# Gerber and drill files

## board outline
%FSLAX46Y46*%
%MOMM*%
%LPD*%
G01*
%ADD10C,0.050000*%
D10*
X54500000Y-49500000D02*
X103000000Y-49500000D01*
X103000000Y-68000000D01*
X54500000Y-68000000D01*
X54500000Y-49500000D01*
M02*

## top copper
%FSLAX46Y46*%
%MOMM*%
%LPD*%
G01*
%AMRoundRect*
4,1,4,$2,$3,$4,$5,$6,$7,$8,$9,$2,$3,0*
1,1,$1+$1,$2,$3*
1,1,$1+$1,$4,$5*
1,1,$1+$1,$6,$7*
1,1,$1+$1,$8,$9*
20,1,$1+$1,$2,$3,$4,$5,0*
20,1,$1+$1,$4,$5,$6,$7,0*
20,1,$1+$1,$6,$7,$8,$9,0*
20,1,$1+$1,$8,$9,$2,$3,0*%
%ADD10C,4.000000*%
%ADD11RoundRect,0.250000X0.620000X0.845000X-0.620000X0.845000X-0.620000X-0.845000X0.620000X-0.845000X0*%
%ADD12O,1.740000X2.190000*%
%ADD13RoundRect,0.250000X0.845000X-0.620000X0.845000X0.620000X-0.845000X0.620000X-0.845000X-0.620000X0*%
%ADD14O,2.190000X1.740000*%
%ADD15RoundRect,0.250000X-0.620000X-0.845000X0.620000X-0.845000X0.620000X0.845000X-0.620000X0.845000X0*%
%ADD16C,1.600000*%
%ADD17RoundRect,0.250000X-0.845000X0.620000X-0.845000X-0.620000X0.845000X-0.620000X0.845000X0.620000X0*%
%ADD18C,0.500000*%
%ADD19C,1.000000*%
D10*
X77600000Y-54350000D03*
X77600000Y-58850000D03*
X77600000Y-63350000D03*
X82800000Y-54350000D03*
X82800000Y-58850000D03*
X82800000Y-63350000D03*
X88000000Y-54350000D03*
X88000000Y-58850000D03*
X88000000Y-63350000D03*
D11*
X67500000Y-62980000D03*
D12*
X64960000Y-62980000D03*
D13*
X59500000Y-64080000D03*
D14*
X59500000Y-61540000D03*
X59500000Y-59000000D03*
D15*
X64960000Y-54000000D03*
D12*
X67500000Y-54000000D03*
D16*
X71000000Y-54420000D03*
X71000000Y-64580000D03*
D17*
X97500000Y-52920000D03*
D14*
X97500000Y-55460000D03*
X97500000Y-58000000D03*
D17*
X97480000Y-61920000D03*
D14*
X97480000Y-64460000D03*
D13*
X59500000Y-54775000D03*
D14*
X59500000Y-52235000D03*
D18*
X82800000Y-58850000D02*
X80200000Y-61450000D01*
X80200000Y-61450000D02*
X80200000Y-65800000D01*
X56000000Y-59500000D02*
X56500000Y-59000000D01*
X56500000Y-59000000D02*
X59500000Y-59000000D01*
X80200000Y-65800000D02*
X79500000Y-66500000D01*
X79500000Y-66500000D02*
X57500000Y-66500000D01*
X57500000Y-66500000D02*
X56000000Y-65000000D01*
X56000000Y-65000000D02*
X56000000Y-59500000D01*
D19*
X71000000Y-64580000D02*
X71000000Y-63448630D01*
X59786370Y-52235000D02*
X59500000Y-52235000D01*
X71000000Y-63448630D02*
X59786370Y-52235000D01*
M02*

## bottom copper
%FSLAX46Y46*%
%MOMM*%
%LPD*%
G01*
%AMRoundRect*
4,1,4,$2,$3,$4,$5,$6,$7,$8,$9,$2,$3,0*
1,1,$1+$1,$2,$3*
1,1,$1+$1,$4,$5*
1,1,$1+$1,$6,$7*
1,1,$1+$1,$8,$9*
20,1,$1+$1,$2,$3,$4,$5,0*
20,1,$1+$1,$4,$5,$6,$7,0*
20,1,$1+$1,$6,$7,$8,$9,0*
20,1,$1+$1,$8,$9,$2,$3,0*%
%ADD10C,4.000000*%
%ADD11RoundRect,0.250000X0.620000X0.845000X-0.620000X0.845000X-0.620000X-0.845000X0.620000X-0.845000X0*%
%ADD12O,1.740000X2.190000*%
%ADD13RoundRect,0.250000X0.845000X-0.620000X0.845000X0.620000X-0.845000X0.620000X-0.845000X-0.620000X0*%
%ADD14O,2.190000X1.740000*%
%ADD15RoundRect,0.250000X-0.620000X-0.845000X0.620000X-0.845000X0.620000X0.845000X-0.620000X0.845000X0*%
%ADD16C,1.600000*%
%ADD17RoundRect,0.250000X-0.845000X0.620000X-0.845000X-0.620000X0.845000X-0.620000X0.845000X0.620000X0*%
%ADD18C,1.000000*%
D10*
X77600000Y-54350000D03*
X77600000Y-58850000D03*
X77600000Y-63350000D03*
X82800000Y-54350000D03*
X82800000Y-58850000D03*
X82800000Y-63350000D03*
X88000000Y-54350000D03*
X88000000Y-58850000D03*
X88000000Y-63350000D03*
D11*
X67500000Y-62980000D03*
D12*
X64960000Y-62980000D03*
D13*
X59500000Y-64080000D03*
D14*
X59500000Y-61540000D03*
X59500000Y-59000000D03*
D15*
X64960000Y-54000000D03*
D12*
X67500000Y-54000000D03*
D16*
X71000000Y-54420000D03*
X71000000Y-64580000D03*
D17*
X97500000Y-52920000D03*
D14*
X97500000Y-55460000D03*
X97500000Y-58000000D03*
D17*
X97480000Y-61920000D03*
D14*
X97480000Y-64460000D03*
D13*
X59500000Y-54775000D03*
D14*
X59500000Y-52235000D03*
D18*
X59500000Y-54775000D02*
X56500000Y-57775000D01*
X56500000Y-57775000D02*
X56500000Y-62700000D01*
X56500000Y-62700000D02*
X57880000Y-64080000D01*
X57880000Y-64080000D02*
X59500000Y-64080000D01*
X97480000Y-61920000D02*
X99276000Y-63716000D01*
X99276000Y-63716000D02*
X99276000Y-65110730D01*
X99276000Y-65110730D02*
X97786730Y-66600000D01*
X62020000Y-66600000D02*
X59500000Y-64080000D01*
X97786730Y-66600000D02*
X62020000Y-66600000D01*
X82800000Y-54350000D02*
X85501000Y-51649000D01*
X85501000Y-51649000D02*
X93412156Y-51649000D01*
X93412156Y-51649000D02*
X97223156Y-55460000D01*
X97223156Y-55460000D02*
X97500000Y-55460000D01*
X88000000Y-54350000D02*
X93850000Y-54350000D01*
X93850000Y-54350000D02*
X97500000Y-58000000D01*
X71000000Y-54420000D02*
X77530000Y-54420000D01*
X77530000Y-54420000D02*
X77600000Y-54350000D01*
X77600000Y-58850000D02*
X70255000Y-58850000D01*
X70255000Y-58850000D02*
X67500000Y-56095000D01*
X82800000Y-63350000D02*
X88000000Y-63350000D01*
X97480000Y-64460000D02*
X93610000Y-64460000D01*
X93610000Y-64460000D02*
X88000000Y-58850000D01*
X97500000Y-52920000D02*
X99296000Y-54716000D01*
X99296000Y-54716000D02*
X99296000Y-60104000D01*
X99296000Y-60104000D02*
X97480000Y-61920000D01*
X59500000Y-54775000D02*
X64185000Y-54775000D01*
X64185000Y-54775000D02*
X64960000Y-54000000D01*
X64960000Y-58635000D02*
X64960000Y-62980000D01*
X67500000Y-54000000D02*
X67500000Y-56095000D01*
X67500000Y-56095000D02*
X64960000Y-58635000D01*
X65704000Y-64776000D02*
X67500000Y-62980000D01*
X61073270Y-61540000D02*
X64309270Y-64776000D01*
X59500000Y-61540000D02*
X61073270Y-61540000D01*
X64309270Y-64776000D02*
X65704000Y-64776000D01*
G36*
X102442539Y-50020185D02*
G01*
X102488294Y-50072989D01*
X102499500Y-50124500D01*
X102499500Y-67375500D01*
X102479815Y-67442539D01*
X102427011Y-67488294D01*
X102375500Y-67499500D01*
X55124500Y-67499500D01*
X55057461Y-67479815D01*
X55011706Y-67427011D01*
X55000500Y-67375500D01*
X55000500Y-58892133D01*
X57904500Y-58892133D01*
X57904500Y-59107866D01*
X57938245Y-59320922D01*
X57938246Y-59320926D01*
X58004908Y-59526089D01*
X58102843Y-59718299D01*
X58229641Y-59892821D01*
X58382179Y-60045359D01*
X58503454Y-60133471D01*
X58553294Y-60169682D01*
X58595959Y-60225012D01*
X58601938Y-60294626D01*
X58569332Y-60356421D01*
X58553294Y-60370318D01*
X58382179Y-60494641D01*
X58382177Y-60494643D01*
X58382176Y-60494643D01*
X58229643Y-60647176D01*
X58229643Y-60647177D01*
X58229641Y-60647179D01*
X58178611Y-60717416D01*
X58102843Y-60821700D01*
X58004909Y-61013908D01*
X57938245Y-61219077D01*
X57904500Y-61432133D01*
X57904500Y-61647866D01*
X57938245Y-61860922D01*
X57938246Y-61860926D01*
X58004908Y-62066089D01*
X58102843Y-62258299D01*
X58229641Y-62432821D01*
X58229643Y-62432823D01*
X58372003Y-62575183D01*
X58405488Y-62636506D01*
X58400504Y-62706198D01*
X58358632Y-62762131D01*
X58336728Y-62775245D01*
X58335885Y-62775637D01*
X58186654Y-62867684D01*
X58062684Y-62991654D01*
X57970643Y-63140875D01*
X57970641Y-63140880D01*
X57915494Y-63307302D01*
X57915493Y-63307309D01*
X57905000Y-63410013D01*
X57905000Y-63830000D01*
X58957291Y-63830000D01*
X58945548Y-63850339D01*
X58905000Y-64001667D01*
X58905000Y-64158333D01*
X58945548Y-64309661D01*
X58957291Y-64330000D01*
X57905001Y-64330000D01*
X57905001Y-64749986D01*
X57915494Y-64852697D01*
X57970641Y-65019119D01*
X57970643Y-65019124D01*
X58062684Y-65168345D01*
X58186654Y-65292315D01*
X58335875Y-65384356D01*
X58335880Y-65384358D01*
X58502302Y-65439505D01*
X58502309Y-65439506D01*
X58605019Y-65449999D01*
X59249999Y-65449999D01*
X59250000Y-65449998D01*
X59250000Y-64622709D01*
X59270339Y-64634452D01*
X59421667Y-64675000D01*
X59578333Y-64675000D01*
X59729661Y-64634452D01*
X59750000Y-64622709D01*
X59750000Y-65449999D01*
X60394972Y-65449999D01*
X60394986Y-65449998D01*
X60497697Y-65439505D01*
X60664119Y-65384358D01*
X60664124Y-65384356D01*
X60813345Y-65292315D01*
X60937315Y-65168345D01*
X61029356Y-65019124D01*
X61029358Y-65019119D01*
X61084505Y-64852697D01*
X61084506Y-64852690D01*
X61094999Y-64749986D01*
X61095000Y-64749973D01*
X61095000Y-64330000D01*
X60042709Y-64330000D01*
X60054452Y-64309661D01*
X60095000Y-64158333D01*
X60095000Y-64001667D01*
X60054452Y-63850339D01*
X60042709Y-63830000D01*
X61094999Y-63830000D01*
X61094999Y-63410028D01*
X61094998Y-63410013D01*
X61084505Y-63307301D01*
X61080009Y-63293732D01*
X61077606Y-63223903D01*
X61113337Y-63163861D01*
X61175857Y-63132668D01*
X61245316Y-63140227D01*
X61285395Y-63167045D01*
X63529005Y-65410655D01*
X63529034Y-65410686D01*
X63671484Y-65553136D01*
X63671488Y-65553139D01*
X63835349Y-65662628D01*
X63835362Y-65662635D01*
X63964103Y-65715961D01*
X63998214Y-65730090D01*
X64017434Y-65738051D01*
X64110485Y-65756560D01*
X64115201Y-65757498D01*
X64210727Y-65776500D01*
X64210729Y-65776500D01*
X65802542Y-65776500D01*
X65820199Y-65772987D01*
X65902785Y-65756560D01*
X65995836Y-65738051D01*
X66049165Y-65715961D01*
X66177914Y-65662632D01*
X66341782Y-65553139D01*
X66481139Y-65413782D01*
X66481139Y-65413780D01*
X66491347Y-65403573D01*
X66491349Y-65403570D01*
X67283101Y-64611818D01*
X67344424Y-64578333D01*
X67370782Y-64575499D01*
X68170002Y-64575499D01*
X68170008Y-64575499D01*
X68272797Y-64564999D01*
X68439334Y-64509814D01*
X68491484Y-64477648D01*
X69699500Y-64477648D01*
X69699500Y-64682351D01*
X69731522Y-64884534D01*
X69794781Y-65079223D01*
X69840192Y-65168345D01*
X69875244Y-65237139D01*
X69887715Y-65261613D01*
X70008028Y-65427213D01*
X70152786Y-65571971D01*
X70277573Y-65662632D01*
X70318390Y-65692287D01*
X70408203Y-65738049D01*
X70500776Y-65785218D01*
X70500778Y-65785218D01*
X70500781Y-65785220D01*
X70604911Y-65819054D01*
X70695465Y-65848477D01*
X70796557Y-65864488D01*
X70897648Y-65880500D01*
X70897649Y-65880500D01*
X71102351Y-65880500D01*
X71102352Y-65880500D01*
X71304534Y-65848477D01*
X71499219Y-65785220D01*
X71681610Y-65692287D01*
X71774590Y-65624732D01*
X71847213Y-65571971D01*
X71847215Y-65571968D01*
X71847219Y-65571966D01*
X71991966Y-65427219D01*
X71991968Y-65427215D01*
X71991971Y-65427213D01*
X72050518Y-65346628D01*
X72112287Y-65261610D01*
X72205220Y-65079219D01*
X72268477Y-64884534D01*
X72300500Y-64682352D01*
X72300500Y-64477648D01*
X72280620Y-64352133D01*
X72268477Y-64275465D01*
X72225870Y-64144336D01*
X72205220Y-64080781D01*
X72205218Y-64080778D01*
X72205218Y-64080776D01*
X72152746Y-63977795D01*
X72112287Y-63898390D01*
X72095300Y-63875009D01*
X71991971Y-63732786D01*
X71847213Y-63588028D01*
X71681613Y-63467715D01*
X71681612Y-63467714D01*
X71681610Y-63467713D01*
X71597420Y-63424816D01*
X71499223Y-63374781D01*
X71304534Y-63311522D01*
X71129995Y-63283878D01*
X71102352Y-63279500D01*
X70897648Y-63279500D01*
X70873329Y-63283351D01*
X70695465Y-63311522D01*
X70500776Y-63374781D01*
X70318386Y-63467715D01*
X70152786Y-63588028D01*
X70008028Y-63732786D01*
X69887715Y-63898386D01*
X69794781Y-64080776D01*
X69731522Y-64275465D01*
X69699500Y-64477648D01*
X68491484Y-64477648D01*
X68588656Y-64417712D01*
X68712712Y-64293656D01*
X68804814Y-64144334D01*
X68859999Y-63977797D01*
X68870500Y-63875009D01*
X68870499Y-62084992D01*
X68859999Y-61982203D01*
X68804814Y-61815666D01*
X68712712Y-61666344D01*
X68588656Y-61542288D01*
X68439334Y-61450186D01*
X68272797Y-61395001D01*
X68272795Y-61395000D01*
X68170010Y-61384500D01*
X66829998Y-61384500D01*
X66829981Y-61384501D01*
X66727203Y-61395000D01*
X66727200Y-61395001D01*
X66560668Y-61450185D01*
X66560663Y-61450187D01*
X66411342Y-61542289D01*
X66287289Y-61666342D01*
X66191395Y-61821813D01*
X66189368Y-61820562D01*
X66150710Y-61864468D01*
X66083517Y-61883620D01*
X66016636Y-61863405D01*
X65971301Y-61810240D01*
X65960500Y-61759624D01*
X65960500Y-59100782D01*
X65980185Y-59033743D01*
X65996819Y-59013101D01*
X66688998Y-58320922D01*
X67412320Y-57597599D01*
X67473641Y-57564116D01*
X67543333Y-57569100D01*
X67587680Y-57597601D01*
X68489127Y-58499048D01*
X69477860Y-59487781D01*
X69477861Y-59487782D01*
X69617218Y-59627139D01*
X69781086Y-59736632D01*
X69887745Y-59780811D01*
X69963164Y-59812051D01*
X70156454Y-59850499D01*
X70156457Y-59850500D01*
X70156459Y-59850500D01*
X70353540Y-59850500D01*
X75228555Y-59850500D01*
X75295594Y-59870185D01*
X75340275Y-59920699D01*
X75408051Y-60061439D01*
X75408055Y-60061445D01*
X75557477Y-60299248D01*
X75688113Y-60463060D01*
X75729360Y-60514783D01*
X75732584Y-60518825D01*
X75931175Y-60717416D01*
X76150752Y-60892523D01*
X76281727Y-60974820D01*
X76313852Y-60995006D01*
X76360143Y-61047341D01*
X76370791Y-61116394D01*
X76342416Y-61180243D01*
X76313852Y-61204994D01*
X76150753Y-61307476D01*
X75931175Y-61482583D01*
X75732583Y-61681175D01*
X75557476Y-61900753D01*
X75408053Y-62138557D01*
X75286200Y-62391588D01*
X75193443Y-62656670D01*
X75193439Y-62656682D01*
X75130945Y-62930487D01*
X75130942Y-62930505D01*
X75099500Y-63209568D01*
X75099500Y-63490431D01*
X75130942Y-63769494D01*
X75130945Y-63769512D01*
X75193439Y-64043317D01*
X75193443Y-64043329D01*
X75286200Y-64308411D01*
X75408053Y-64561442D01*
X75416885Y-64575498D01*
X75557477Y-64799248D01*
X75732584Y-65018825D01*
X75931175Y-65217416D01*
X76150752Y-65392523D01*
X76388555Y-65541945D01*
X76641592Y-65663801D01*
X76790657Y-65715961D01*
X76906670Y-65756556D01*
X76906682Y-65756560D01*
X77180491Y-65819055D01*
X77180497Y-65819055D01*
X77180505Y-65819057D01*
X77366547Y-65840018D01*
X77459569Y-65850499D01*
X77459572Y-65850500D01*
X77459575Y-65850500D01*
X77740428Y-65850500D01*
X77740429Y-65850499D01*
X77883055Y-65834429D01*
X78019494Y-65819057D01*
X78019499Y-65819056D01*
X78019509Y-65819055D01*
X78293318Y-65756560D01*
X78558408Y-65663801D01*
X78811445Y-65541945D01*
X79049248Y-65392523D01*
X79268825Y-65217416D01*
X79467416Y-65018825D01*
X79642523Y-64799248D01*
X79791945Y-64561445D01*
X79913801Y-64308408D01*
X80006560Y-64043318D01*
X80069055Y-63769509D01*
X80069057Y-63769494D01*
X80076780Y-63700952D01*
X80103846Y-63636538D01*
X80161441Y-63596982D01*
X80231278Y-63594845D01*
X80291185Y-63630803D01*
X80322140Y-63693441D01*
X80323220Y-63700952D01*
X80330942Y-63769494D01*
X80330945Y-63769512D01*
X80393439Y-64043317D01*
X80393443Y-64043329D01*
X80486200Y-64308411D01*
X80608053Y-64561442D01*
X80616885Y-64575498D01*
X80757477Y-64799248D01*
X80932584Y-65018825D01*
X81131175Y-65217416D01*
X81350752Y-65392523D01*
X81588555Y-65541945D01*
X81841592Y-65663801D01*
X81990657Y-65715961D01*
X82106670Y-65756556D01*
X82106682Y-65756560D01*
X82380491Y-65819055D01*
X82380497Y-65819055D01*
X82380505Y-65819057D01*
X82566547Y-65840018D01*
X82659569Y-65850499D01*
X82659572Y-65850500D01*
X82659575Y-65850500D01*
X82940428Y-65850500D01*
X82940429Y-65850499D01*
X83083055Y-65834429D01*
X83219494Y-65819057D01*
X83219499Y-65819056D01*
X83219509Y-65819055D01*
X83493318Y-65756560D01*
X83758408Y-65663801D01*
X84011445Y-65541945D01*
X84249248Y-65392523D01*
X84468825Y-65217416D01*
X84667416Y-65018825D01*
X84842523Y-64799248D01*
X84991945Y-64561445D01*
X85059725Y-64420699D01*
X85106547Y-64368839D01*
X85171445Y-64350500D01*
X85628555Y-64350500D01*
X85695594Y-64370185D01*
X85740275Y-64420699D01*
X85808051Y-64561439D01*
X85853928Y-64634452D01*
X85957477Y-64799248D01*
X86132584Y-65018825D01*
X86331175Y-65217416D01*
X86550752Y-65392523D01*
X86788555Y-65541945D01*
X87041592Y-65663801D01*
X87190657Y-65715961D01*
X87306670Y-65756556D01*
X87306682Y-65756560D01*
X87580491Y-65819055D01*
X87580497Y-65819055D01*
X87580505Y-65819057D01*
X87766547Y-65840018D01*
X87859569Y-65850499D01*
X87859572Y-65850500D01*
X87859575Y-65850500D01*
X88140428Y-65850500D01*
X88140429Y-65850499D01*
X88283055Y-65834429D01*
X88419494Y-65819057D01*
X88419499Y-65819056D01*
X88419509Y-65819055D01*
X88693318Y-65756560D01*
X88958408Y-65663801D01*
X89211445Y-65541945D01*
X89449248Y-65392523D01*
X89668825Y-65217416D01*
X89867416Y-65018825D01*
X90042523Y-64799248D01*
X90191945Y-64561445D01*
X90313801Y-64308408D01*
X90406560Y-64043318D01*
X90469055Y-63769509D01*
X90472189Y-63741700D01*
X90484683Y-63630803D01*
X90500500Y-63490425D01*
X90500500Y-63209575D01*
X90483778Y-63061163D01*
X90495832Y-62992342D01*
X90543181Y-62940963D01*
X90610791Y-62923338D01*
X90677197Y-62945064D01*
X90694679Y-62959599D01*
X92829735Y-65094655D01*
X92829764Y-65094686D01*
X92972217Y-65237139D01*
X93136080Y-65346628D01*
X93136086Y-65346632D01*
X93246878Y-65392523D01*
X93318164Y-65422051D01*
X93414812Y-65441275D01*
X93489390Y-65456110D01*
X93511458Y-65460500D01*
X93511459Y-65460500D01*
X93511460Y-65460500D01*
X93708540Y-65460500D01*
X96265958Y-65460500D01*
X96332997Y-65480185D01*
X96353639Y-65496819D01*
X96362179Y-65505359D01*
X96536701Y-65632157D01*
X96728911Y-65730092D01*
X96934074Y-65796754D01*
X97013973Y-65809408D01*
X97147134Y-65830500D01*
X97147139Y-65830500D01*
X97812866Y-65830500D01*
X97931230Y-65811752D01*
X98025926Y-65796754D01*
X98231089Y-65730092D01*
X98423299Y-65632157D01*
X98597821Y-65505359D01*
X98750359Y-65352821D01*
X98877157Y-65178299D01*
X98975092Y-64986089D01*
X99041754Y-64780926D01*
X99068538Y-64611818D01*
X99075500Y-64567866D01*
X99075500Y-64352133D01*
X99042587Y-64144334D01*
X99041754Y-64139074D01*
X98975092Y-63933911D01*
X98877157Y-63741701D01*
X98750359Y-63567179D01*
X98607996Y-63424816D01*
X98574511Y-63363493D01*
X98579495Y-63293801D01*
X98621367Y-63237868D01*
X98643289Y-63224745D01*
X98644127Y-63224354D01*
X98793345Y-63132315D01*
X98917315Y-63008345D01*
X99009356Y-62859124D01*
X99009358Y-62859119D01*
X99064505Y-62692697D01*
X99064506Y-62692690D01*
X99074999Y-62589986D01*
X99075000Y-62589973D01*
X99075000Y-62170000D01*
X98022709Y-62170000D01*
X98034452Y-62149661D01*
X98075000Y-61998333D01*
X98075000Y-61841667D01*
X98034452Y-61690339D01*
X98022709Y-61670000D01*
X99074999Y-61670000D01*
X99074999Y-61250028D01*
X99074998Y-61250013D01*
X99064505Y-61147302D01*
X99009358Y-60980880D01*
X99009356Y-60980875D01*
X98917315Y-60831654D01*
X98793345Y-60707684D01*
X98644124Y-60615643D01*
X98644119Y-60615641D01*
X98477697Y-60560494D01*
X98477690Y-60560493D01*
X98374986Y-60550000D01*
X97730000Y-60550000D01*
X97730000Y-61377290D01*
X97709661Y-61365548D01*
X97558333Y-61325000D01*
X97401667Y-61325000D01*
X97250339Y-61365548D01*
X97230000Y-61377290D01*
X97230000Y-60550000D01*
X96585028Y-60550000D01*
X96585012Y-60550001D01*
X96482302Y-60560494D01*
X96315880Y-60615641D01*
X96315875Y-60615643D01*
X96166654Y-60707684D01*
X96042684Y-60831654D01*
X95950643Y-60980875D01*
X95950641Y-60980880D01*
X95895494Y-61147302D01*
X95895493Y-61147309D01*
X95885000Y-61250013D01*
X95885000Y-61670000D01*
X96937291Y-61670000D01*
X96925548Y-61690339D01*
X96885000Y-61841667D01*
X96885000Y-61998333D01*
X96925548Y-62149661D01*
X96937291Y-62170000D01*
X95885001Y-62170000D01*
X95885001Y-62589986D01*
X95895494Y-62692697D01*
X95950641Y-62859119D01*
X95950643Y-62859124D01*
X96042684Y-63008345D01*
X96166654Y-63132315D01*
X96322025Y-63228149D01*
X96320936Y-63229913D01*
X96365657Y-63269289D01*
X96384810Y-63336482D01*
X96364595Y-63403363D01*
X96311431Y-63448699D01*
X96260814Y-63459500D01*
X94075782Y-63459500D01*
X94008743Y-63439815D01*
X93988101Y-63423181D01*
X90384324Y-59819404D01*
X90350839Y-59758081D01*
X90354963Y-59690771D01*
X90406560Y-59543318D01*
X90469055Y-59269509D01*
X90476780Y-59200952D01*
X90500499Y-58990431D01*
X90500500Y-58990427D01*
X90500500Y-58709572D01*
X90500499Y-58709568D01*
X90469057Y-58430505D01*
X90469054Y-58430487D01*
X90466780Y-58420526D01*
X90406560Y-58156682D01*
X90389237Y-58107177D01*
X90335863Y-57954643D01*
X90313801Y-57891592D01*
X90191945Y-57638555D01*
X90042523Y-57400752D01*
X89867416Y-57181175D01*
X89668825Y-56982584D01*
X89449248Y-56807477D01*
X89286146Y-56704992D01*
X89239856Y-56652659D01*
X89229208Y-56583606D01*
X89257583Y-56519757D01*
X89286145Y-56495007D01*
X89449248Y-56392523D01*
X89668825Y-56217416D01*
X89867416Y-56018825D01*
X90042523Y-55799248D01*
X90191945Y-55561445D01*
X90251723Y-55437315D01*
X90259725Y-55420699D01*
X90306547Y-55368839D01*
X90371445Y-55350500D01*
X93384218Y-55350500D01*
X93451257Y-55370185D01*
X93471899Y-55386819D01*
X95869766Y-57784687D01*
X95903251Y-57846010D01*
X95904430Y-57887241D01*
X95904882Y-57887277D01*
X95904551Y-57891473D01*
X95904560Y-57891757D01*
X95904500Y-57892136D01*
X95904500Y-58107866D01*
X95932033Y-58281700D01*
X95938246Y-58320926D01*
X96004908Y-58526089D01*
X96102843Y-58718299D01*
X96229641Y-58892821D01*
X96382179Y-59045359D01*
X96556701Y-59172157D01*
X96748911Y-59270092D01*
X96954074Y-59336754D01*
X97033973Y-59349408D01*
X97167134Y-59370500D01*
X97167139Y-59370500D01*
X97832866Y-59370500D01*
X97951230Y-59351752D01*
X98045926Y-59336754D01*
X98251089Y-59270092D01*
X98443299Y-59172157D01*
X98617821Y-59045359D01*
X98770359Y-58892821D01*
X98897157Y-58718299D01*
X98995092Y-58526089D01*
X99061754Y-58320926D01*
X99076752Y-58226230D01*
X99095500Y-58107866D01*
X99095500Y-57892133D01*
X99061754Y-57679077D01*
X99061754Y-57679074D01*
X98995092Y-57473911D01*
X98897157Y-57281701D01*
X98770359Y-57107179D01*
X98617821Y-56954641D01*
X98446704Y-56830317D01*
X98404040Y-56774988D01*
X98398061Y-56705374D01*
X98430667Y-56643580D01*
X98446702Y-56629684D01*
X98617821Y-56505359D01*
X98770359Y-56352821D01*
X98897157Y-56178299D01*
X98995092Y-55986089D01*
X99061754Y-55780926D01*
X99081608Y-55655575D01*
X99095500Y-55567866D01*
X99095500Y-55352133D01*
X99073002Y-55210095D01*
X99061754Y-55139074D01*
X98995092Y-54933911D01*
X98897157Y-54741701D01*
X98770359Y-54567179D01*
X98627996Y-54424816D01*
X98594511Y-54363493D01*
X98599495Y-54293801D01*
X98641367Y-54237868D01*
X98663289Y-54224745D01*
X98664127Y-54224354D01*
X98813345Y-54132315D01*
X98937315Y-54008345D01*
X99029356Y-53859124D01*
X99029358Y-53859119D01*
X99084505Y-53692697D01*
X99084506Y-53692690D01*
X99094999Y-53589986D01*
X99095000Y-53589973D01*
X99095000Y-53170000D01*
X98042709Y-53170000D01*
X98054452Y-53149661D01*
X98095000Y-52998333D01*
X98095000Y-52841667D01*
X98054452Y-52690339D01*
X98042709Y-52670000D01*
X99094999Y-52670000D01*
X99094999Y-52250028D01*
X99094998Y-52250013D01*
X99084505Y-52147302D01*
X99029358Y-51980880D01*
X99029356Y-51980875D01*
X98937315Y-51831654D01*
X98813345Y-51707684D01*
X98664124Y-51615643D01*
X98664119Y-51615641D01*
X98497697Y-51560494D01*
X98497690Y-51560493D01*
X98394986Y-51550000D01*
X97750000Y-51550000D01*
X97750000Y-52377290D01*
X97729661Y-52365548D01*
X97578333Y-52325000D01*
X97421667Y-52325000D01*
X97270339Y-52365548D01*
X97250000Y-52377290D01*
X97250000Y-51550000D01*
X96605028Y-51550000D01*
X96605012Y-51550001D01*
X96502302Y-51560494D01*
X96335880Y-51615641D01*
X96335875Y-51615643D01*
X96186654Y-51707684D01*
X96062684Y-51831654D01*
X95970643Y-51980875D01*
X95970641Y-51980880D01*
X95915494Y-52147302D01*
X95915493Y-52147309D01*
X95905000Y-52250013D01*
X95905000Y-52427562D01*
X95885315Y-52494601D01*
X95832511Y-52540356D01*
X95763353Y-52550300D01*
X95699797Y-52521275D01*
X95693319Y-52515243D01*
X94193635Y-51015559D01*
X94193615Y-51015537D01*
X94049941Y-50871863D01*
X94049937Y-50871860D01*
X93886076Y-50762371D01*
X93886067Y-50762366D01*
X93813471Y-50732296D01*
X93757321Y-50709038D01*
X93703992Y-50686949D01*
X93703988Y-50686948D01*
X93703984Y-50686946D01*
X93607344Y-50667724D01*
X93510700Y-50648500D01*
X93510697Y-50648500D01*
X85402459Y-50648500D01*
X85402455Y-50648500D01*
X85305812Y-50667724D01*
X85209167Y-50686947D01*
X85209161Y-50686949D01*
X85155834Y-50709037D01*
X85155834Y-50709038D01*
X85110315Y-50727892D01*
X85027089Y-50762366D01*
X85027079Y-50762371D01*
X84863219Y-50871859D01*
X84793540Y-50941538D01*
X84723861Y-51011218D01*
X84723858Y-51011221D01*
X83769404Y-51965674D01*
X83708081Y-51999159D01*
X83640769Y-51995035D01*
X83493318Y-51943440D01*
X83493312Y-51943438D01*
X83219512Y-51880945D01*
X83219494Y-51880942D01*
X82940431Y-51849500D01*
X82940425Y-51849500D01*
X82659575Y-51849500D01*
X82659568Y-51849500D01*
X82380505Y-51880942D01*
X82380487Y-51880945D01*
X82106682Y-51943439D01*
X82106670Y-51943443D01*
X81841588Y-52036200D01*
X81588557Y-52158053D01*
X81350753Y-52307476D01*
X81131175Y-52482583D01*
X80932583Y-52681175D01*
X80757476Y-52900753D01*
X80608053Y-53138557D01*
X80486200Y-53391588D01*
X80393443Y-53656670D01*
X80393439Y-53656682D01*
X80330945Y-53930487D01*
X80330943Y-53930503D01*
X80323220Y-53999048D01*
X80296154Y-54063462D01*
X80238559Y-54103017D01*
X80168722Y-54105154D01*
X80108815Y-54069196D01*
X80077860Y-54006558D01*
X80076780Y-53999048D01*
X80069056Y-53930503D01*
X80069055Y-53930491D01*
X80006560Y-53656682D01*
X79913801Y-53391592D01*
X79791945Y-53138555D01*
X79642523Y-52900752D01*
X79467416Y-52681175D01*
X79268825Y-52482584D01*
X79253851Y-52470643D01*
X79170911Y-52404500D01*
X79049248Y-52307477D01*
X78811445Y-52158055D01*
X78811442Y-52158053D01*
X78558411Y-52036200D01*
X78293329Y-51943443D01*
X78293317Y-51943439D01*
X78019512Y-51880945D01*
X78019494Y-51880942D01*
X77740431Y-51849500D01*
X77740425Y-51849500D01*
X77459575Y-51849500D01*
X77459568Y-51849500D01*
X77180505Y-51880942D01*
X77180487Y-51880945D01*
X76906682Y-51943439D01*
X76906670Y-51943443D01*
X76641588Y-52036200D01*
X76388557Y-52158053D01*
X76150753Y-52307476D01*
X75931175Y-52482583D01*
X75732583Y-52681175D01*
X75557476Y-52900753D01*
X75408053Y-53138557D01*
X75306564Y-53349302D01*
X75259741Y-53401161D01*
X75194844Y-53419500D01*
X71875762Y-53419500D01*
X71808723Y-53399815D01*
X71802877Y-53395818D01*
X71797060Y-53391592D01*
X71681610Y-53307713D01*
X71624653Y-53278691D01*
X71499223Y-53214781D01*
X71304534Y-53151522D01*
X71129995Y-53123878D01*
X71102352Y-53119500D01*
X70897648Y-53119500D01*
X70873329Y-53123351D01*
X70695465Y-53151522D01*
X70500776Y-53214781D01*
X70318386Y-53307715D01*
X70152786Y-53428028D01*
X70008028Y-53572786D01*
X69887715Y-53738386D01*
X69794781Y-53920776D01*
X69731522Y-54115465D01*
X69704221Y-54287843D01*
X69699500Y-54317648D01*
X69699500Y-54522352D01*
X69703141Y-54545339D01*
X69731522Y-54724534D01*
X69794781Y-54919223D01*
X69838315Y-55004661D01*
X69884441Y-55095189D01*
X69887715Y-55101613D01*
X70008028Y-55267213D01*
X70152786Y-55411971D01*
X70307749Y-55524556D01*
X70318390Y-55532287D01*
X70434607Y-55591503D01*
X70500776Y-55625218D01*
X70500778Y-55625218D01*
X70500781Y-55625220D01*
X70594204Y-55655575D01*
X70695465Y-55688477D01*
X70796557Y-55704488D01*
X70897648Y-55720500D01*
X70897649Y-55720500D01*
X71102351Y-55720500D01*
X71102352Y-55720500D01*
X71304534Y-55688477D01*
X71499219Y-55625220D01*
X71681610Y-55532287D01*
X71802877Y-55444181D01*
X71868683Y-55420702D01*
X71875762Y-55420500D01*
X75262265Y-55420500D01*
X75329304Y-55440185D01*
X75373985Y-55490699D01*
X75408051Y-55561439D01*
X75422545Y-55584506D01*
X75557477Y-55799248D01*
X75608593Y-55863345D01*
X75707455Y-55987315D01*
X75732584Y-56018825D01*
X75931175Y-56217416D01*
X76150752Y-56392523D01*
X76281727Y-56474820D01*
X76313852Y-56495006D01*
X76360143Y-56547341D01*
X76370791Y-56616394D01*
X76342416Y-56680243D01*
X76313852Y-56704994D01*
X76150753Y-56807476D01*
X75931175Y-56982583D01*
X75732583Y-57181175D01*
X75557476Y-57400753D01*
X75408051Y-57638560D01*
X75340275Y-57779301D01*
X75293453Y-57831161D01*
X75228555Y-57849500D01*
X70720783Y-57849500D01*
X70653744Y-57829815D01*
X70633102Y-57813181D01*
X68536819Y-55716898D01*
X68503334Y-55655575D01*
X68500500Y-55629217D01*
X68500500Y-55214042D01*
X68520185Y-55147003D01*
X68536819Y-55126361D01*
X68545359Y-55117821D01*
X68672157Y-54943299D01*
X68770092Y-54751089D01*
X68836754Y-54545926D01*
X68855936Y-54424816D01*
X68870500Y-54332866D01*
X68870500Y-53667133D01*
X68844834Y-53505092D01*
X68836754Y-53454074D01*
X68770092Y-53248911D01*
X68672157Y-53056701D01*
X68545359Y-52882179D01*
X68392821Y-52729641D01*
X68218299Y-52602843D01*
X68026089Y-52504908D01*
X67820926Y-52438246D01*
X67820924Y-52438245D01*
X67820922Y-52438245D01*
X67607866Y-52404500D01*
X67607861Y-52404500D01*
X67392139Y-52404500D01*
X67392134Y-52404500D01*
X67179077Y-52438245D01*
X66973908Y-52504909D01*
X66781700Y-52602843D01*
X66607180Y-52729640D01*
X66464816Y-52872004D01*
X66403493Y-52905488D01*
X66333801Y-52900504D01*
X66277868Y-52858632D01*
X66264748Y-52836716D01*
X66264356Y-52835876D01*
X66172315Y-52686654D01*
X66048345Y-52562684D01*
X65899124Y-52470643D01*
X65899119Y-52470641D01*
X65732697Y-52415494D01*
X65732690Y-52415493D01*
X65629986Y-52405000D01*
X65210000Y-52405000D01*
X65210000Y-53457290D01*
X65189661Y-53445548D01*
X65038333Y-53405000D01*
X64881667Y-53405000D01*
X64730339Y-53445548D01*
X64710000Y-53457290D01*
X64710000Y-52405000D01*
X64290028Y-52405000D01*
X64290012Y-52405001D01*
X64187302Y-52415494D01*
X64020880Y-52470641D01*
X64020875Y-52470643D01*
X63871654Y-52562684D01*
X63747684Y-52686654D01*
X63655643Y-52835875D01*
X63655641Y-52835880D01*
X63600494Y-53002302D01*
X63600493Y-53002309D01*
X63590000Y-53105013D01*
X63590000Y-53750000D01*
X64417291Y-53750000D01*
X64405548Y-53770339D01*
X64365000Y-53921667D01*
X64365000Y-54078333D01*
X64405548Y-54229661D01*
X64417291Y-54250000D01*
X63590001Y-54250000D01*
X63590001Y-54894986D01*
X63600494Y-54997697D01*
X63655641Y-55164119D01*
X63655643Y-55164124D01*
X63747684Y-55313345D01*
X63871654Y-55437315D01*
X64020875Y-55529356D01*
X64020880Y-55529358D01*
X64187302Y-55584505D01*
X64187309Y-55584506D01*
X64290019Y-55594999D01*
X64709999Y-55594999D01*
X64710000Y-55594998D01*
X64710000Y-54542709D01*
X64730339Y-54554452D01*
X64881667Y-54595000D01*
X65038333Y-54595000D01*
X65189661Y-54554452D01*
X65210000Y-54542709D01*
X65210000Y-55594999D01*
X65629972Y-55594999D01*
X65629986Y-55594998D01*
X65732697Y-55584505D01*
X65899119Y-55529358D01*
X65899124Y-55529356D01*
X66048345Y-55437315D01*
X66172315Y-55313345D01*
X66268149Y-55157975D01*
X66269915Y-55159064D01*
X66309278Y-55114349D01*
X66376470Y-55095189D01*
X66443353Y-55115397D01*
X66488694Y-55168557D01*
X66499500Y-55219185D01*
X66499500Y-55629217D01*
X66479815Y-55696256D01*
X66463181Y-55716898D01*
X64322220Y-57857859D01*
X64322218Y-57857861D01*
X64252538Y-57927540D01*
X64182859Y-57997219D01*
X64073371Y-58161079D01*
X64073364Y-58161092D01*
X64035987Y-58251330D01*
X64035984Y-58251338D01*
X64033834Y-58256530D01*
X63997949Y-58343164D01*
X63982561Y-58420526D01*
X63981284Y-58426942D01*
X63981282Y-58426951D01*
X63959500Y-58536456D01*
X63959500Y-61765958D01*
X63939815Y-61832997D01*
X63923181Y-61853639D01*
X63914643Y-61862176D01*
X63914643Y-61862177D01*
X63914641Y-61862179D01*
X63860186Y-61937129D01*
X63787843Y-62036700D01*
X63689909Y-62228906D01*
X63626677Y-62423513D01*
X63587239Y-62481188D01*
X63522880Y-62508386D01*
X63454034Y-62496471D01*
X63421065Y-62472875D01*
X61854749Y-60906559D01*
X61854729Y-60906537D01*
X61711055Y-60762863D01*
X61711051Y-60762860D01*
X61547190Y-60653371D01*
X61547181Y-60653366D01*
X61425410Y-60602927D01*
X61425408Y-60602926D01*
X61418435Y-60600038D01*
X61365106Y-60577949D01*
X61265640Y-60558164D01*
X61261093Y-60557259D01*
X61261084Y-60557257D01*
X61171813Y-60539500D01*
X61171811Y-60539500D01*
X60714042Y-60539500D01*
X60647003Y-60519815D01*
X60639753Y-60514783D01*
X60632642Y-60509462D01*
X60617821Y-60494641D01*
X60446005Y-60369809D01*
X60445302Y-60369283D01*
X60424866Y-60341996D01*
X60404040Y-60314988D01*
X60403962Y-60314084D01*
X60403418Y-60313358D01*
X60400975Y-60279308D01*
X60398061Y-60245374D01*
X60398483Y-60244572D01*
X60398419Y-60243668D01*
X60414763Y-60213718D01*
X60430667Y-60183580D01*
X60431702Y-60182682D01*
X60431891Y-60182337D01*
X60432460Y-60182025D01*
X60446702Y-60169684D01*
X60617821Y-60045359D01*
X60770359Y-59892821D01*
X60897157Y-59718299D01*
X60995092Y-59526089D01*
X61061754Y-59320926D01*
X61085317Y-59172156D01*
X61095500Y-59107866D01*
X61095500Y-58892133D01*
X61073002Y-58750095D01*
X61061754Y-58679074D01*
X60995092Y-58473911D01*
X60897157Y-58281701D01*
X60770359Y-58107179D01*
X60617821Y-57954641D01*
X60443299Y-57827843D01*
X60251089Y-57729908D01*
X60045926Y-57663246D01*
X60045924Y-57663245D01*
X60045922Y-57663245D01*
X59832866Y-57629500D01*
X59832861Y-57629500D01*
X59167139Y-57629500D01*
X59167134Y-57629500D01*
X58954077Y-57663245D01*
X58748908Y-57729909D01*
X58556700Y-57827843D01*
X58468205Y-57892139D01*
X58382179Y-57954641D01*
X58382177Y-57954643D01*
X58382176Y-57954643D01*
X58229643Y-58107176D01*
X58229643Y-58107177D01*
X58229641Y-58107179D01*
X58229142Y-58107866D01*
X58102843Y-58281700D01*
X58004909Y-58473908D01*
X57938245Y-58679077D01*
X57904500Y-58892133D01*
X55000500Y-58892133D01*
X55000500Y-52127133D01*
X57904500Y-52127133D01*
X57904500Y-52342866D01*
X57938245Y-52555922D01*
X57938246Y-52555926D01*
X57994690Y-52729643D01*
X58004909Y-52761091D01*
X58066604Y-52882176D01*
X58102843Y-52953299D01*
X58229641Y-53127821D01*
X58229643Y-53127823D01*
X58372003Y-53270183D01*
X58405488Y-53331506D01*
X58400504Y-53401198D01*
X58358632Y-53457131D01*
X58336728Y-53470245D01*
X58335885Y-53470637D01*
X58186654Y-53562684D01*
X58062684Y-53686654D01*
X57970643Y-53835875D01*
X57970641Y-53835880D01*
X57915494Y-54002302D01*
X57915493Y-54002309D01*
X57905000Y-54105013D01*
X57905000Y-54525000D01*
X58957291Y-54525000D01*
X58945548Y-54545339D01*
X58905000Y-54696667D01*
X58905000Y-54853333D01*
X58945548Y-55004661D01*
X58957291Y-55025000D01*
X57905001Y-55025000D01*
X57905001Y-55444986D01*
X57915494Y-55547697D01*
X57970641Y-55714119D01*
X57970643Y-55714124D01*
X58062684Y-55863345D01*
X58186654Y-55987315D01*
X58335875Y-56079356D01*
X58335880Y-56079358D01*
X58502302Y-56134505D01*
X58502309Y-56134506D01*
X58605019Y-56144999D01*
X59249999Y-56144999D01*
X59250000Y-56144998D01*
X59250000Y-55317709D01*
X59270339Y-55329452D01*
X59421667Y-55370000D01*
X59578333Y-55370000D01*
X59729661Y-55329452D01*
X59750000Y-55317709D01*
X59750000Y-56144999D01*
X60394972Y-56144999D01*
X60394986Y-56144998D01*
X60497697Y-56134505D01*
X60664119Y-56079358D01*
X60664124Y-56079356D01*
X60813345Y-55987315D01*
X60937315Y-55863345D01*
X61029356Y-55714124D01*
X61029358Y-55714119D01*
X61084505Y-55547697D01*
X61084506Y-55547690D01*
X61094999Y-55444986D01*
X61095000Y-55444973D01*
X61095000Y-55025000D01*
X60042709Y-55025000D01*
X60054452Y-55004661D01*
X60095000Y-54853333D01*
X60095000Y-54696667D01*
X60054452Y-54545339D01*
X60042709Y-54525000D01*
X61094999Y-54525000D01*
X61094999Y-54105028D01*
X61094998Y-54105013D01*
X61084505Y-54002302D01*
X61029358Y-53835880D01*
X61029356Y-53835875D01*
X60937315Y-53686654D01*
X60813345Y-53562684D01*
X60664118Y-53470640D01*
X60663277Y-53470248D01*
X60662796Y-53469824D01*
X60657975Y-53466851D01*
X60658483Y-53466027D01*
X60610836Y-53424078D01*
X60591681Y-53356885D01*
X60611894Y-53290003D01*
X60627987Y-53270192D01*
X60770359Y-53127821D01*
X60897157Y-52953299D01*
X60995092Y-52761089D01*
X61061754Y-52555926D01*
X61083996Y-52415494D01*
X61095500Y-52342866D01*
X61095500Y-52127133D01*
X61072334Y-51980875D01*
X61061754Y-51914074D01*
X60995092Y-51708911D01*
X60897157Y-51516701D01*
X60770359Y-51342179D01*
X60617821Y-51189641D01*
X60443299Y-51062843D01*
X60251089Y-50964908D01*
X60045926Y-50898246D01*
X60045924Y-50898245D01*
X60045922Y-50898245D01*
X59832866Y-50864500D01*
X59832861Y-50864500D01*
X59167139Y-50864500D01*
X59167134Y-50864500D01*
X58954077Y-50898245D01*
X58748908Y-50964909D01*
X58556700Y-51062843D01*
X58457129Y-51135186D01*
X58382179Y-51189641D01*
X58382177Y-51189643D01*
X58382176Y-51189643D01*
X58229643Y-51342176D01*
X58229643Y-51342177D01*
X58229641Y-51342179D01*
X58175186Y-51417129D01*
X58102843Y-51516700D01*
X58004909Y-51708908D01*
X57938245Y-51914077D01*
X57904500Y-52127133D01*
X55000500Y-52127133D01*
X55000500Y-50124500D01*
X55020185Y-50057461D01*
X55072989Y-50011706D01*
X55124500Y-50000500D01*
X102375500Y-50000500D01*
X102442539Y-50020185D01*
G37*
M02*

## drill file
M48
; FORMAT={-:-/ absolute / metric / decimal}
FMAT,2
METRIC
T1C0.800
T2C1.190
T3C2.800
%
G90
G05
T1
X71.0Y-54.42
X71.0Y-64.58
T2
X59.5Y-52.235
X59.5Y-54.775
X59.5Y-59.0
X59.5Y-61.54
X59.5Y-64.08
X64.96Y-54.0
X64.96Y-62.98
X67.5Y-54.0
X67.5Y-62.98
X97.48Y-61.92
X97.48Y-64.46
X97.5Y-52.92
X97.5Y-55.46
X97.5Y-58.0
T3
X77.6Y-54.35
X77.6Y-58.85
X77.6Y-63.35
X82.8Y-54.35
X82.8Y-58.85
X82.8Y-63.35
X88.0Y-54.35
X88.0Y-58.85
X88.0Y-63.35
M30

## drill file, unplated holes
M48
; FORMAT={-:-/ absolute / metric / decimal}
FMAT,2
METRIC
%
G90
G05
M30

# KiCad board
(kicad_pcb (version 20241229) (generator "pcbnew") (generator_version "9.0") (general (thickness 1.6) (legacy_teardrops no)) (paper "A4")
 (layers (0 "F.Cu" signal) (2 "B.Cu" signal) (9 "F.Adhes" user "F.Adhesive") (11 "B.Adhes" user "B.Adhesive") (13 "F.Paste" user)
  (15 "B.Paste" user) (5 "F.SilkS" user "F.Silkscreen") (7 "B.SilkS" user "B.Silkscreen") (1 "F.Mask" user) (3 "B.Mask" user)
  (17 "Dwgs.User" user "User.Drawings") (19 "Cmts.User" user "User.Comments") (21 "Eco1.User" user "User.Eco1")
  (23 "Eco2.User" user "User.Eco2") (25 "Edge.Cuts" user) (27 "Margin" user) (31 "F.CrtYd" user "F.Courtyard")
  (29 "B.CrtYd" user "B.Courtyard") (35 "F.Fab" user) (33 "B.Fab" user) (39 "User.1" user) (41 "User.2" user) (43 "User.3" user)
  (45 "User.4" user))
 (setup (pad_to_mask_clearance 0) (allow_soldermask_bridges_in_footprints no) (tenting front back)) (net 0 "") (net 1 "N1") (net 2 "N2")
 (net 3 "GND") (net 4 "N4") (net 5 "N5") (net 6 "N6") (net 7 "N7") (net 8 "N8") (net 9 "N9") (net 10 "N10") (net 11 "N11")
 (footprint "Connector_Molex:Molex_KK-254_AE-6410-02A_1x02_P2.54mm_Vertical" (layer "F.Cu") (at 67.5 62.98 180)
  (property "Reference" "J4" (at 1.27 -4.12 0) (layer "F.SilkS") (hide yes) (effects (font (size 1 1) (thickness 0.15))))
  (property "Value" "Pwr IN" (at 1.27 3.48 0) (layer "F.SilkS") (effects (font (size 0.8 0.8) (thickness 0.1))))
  (pad "1" thru_hole roundrect (at 0 0 180) (size 1.74 2.19) (drill 1.19) (layers "*.Cu" "*.Mask") (remove_unused_layers no)
   (roundrect_rratio 0.143678) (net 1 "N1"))
  (pad "2" thru_hole oval (at 2.54 0 180) (size 1.74 2.19) (drill 1.19) (layers "*.Cu" "*.Mask") (remove_unused_layers no) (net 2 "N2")))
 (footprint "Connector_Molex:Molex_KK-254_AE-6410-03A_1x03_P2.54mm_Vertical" (layer "F.Cu") (at 59.5 64.08 90)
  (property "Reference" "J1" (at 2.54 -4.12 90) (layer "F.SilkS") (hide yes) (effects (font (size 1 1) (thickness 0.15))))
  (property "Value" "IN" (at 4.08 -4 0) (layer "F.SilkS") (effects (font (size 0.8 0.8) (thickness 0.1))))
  (pad "1" thru_hole roundrect (at 0 0 90) (size 1.74 2.19) (drill 1.19) (layers "*.Cu" "*.Mask") (remove_unused_layers no)
   (roundrect_rratio 0.143678) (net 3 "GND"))
  (pad "2" thru_hole oval (at 2.54 0 90) (size 1.74 2.19) (drill 1.19) (layers "*.Cu" "*.Mask") (remove_unused_layers no) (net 1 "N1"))
  (pad "3" thru_hole oval (at 5.08 0 90) (size 1.74 2.19) (drill 1.19) (layers "*.Cu" "*.Mask") (remove_unused_layers no) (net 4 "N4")))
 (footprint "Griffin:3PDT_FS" (layer "F.Cu") (at 80.6 57.85)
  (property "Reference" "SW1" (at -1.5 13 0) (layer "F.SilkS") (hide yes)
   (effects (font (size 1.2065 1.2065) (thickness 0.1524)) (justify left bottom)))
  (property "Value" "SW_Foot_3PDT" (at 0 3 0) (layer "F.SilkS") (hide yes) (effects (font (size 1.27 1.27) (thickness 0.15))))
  (pad "A1" thru_hole circle (at -3 -3.5 180) (size 4 4) (drill 2.8) (layers "*.Cu" "*.Mask") (remove_unused_layers no) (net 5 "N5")
   (solder_mask_margin 0.1016))
  (pad "A2" thru_hole circle (at -3 1 180) (size 4 4) (drill 2.8) (layers "*.Cu" "*.Mask") (remove_unused_layers no) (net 2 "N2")
   (solder_mask_margin 0.1016))
  (pad "A3" thru_hole circle (at -3 5.5 180) (size 4 4) (drill 2.8) (layers "*.Cu" "*.Mask") (remove_unused_layers no) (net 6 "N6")
   (solder_mask_margin 0.1016))
  (pad "B1" thru_hole circle (at 2.2 -3.5 180) (size 4 4) (drill 2.8) (layers "*.Cu" "*.Mask") (remove_unused_layers no) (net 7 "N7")
   (solder_mask_margin 0.1016))
  (pad "B2" thru_hole circle (at 2.2 1 180) (size 4 4) (drill 2.8) (layers "*.Cu" "*.Mask") (remove_unused_layers no) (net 4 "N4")
   (solder_mask_margin 0.1016))
  (pad "B3" thru_hole circle (at 2.2 5.5 180) (size 4 4) (drill 2.8) (layers "*.Cu" "*.Mask") (remove_unused_layers no) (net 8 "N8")
   (solder_mask_margin 0.1016))
  (pad "C1" thru_hole circle (at 7.4 -3.5 180) (size 4 4) (drill 2.8) (layers "*.Cu" "*.Mask") (remove_unused_layers no) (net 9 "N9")
   (solder_mask_margin 0.1016))
  (pad "C2" thru_hole circle (at 7.4 1 180) (size 4 4) (drill 2.8) (layers "*.Cu" "*.Mask") (remove_unused_layers no) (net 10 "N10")
   (solder_mask_margin 0.1016))
  (pad "C3" thru_hole circle (at 7.4 5.5 180) (size 4 4) (drill 2.8) (layers "*.Cu" "*.Mask") (remove_unused_layers no) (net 8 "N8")
   (solder_mask_margin 0.1016)))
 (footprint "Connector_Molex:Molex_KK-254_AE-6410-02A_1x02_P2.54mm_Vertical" (layer "F.Cu") (at 64.96 54)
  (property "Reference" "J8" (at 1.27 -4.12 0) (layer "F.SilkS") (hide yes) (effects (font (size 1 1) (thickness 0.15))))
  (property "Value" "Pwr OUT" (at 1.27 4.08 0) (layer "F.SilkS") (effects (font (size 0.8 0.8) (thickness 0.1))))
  (pad "1" thru_hole roundrect (at 0 0) (size 1.74 2.19) (drill 1.19) (layers "*.Cu" "*.Mask") (remove_unused_layers no)
   (roundrect_rratio 0.143678) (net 3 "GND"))
  (pad "2" thru_hole oval (at 2.54 0) (size 1.74 2.19) (drill 1.19) (layers "*.Cu" "*.Mask") (remove_unused_layers no) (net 2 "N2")))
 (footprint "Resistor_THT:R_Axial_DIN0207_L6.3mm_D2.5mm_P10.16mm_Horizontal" (layer "F.Cu") (at 71 54.42 -90)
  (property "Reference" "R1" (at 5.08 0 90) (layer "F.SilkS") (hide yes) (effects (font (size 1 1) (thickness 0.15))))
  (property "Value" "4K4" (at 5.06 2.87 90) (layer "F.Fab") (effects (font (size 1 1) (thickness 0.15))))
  (pad "1" thru_hole circle (at 0 0 270) (size 1.6 1.6) (drill 0.8) (layers "*.Cu" "*.Mask") (remove_unused_layers no) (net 5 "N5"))
  (pad "2" thru_hole circle (at 10.16 0 270) (size 1.6 1.6) (drill 0.8) (layers "*.Cu" "*.Mask") (remove_unused_layers no) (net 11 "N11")))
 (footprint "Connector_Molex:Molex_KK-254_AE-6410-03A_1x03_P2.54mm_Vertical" (layer "F.Cu") (at 97.5 52.92 -90)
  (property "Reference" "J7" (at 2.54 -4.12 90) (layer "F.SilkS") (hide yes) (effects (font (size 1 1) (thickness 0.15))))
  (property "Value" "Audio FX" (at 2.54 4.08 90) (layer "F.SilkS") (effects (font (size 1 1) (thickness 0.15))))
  (pad "1" thru_hole roundrect (at 0 0 270) (size 1.74 2.19) (drill 1.19) (layers "*.Cu" "*.Mask") (remove_unused_layers no)
   (roundrect_rratio 0.143678) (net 3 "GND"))
  (pad "2" thru_hole oval (at 2.54 0 270) (size 1.74 2.19) (drill 1.19) (layers "*.Cu" "*.Mask") (remove_unused_layers no) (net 7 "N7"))
  (pad "3" thru_hole oval (at 5.08 0 270) (size 1.74 2.19) (drill 1.19) (layers "*.Cu" "*.Mask") (remove_unused_layers no) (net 9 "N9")))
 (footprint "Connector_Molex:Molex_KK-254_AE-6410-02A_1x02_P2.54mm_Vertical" (layer "F.Cu") (at 97.48 61.92 -90)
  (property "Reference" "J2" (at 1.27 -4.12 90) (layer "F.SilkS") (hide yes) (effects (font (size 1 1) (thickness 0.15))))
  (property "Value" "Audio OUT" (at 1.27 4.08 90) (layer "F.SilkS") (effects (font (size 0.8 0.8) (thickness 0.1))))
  (pad "1" thru_hole roundrect (at 0 0 270) (size 1.74 2.19) (drill 1.19) (layers "*.Cu" "*.Mask") (remove_unused_layers no)
   (roundrect_rratio 0.143678) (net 3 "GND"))
  (pad "2" thru_hole oval (at 2.54 0 270) (size 1.74 2.19) (drill 1.19) (layers "*.Cu" "*.Mask") (remove_unused_layers no) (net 10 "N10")))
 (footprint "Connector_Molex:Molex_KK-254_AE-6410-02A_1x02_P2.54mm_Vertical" (layer "F.Cu") (at 59.5 54.775 90)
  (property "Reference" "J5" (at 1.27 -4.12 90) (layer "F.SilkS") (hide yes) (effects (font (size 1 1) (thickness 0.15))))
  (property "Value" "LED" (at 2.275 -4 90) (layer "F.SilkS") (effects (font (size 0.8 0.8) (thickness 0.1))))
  (pad "1" thru_hole roundrect (at 0 0 90) (size 1.74 2.19) (drill 1.19) (layers "*.Cu" "*.Mask") (remove_unused_layers no)
   (roundrect_rratio 0.143678) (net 3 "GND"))
  (pad "2" thru_hole oval (at 2.54 0 90) (size 1.74 2.19) (drill 1.19) (layers "*.Cu" "*.Mask") (remove_unused_layers no) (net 11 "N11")))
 (gr_rect (start 54.5 49.5) (end 103 68) (stroke (width 0.05) (type default)) (fill no) (layer "Edge.Cuts"))
 (segment (start 97.5 52.92) (end 99.296 54.716) (width 1) (layer "B.Cu") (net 3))
 (segment (start 59.5 54.775) (end 56.5 57.775) (width 1) (layer "B.Cu") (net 3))
 (segment (start 59.5 54.775) (end 64.185 54.775) (width 1) (layer "B.Cu") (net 3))
 (segment (start 97.78673 66.6) (end 62.02 66.6) (width 1) (layer "B.Cu") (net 3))
 (segment (start 57.88 64.08) (end 59.5 64.08) (width 1) (layer "B.Cu") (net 3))
 (segment (start 99.296 60.104) (end 97.48 61.92) (width 1) (layer "B.Cu") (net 3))
 (segment (start 56.5 62.7) (end 57.88 64.08) (width 1) (layer "B.Cu") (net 3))
 (segment (start 99.296 54.716) (end 99.296 60.104) (width 1) (layer "B.Cu") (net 3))
 (segment (start 62.02 66.6) (end 59.5 64.08) (width 1) (layer "B.Cu") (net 3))
 (segment (start 97.48 61.92) (end 99.276 63.716) (width 1) (layer "B.Cu") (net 3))
 (segment (start 99.276 65.11073) (end 97.78673 66.6) (width 1) (layer "B.Cu") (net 3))
 (segment (start 56.5 57.775) (end 56.5 62.7) (width 1) (layer "B.Cu") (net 3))
 (segment (start 64.185 54.775) (end 64.96 54) (width 1) (layer "B.Cu") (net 3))
 (segment (start 99.276 63.716) (end 99.276 65.11073) (width 1) (layer "B.Cu") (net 3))
 (segment (start 64.96 58.635) (end 64.96 62.98) (width 1) (layer "B.Cu") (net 2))
 (segment (start 67.5 54) (end 67.5 56.095) (width 1) (layer "B.Cu") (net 2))
 (segment (start 70.255 58.85) (end 67.5 56.095) (width 1) (layer "B.Cu") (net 2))
 (segment (start 67.5 56.095) (end 64.96 58.635) (width 1) (layer "B.Cu") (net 2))
 (segment (start 77.6 58.85) (end 70.255 58.85) (width 1) (layer "B.Cu") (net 2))
 (segment (start 71 64.58) (end 71 63.44863) (width 1) (layer "F.Cu") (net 11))
 (segment (start 59.78637 52.235) (end 59.5 52.235) (width 1) (layer "F.Cu") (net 11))
 (segment (start 71 63.44863) (end 59.78637 52.235) (width 1) (layer "F.Cu") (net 11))
 (segment (start 97.223156 55.46) (end 97.5 55.46) (width 1) (layer "B.Cu") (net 7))
 (segment (start 85.501 51.649) (end 93.412156 51.649) (width 1) (layer "B.Cu") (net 7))
 (segment (start 93.412156 51.649) (end 97.223156 55.46) (width 1) (layer "B.Cu") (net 7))
 (segment (start 82.8 54.35) (end 85.501 51.649) (width 1) (layer "B.Cu") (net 7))
 (segment (start 77.53 54.42) (end 77.6 54.35) (width 1) (layer "B.Cu") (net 5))
 (segment (start 71 54.42) (end 77.53 54.42) (width 1) (layer "B.Cu") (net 5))
 (segment (start 82.8 58.85) (end 80.2 61.45) (width 0.5) (layer "F.Cu") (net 4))
 (segment (start 56 59.5) (end 56.5 59) (width 0.5) (layer "F.Cu") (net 4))
 (segment (start 56.5 59) (end 59.5 59) (width 0.5) (layer "F.Cu") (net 4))
 (segment (start 57.5 66.5) (end 56 65) (width 0.5) (layer "F.Cu") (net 4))
 (segment (start 79.5 66.5) (end 57.5 66.5) (width 0.5) (layer "F.Cu") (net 4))
 (segment (start 80.2 65.8) (end 79.5 66.5) (width 0.5) (layer "F.Cu") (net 4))
 (segment (start 80.2 61.45) (end 80.2 65.8) (width 0.5) (layer "F.Cu") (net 4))
 (segment (start 56 65) (end 56 59.5) (width 0.5) (layer "F.Cu") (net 4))
 (segment (start 65.704 64.776) (end 67.5 62.98) (width 1) (layer "B.Cu") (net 1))
 (segment (start 61.07327 61.54) (end 64.30927 64.776) (width 1) (layer "B.Cu") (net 1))
 (segment (start 59.5 61.54) (end 61.07327 61.54) (width 1) (layer "B.Cu") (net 1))
 (segment (start 64.30927 64.776) (end 65.704 64.776) (width 1) (layer "B.Cu") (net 1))
 (segment (start 93.61 64.46) (end 88 58.85) (width 1) (layer "B.Cu") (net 10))
 (segment (start 97.48 64.46) (end 93.61 64.46) (width 1) (layer "B.Cu") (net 10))
 (segment (start 93.85 54.35) (end 97.5 58) (width 1) (layer "B.Cu") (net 9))
 (segment (start 88 54.35) (end 93.85 54.35) (width 1) (layer "B.Cu") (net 9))
 (segment (start 82.8 63.35) (end 88 63.35) (width 1) (layer "B.Cu") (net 8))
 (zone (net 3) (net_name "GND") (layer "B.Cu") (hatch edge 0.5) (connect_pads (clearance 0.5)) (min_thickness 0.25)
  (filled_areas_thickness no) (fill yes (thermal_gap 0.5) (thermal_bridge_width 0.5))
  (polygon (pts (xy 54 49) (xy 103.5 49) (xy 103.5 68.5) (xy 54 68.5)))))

